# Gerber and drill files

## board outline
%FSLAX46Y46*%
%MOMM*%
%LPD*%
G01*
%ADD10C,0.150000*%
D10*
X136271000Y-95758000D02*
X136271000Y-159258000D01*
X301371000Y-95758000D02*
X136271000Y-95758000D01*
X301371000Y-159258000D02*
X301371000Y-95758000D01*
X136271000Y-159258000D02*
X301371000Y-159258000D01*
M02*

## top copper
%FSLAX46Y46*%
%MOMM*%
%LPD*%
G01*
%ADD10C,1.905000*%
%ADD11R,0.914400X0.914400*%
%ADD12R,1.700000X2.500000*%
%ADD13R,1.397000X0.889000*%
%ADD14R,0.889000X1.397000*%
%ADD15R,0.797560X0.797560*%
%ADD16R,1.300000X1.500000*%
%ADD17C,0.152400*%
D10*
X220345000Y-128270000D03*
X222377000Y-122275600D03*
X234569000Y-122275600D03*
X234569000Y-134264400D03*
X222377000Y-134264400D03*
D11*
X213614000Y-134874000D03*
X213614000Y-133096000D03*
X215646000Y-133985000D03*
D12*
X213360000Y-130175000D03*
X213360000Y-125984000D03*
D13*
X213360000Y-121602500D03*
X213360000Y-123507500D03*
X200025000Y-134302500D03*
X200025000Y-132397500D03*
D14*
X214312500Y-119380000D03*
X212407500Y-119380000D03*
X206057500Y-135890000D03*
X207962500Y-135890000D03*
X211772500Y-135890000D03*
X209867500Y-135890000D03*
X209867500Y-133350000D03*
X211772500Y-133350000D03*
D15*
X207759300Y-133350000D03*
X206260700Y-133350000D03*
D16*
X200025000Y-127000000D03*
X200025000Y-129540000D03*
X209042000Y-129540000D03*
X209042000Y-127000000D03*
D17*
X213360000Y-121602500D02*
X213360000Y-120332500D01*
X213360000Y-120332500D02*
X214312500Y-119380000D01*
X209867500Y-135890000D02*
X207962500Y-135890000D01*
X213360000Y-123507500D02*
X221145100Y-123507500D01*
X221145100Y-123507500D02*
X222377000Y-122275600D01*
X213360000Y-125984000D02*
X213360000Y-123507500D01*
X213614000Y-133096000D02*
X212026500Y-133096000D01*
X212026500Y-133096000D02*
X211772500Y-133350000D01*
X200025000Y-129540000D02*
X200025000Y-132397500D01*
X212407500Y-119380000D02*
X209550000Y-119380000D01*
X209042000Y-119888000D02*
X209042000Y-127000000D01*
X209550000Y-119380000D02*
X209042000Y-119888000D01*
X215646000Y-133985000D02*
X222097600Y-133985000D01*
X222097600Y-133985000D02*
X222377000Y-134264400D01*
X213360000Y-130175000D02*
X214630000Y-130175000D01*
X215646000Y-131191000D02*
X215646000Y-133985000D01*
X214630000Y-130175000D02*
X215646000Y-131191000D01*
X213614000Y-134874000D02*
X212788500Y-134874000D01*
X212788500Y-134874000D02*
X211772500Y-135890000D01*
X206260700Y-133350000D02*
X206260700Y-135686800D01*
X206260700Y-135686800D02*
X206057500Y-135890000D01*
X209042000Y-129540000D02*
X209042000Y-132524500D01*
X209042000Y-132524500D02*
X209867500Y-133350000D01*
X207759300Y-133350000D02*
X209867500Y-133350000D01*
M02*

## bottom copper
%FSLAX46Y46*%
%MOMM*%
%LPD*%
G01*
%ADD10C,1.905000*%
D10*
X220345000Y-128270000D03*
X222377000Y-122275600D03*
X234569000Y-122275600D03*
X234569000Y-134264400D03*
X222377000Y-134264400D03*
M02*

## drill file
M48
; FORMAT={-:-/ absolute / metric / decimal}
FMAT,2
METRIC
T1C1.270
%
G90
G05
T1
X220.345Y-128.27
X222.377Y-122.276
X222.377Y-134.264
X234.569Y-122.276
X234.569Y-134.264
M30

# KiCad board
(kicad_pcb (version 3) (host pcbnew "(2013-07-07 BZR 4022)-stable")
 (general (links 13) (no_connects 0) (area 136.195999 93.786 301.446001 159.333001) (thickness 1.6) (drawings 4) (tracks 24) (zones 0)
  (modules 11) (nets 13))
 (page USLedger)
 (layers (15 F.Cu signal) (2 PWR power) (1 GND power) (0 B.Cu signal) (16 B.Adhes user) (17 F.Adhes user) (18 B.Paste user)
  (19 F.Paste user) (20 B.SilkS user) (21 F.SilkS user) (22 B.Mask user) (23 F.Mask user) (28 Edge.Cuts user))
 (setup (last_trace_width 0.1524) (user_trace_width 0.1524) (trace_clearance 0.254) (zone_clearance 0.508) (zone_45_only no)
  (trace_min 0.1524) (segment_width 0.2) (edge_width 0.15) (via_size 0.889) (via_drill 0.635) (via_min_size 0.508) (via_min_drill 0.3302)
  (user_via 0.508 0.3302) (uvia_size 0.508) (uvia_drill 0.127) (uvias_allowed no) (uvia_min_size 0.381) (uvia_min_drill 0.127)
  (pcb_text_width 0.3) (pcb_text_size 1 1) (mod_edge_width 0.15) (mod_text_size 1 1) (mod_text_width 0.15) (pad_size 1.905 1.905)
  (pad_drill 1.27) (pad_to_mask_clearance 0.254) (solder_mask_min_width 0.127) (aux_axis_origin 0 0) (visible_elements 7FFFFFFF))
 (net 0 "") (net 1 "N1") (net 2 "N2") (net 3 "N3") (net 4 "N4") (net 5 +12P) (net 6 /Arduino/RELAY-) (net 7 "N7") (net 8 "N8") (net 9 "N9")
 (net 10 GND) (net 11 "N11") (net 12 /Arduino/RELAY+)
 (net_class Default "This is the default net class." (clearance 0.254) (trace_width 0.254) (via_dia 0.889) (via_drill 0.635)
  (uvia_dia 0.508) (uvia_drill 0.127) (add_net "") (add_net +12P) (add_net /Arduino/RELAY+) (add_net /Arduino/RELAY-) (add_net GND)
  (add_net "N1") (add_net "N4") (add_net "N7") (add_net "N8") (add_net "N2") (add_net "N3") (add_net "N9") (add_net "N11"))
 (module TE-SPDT (layer F.Cu) (at 220.345 128.27)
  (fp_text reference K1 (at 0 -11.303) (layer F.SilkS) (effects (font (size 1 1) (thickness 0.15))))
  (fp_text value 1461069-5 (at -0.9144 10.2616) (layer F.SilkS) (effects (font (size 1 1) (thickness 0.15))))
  (pad 1 thru_hole circle (at 0 0) (size 1.905 1.905) (drill 1.27) (layers *.Cu *.Mask F.SilkS))
  (pad 2 thru_hole circle (at 2.032 -5.9944) (size 1.905 1.905) (drill 1.27) (layers *.Cu *.Mask F.SilkS) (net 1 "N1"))
  (pad 3 thru_hole circle (at 14.224 -5.9944) (size 1.905 1.905) (drill 1.27) (layers *.Cu *.Mask F.SilkS))
  (pad 4 thru_hole circle (at 14.224 5.9944) (size 1.905 1.905) (drill 1.27) (layers *.Cu *.Mask F.SilkS))
  (pad 5 thru_hole circle (at 2.032 5.9944) (size 1.905 1.905) (drill 1.27) (layers *.Cu *.Mask F.SilkS) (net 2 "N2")))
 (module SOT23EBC (layer F.Cu) (at 214.63 133.985 90)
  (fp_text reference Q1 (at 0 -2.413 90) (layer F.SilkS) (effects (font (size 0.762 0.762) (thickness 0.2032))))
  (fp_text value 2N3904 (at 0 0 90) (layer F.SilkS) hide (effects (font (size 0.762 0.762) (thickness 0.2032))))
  (pad 1 smd rect (at -0.889 -1.016 90) (size 0.9144 0.9144) (layers F.Cu F.Paste F.Mask) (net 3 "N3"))
  (pad 2 smd rect (at 0.889 -1.016 90) (size 0.9144 0.9144) (layers F.Cu F.Paste F.Mask) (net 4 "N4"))
  (pad 3 smd rect (at 0 1.016 90) (size 0.9144 0.9144) (layers F.Cu F.Paste F.Mask) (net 2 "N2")))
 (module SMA (layer F.Cu) (at 213.36 130.175 90)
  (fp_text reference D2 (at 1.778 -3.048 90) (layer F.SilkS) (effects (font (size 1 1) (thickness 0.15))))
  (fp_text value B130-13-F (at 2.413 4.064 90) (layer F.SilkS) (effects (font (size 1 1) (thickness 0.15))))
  (pad 1 smd rect (at 0 0 90) (size 2.5 1.7) (layers F.Cu F.Paste F.Mask) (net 2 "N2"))
  (pad 2 smd rect (at 4.191 0 90) (size 2.5 1.7) (layers F.Cu F.Paste F.Mask) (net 1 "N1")))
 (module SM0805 (layer F.Cu) (at 213.36 122.555 270)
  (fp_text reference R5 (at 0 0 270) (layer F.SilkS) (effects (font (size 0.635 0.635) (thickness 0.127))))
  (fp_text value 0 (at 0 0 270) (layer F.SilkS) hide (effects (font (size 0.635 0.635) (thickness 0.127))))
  (pad 1 smd rect (at -0.9525 0 270) (size 0.889 1.397) (layers F.Cu F.Paste F.Mask) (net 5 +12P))
  (pad 2 smd rect (at 0.9525 0 270) (size 0.889 1.397) (layers F.Cu F.Paste F.Mask) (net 1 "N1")))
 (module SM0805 (layer F.Cu) (at 200.025 133.35 90)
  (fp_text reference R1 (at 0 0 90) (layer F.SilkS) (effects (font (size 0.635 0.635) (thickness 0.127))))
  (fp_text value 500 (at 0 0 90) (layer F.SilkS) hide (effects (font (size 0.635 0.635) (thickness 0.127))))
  (pad 1 smd rect (at -0.9525 0 90) (size 0.889 1.397) (layers F.Cu F.Paste F.Mask) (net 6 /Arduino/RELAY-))
  (pad 2 smd rect (at 0.9525 0 90) (size 0.889 1.397) (layers F.Cu F.Paste F.Mask) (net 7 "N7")))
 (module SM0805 (layer F.Cu) (at 213.36 119.38 180)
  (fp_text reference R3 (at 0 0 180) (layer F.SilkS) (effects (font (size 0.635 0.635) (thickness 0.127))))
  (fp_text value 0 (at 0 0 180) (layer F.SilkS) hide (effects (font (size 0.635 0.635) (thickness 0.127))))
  (pad 1 smd rect (at -0.9525 0 180) (size 0.889 1.397) (layers F.Cu F.Paste F.Mask) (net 5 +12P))
  (pad 2 smd rect (at 0.9525 0 180) (size 0.889 1.397) (layers F.Cu F.Paste F.Mask) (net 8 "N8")))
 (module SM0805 (layer F.Cu) (at 207.01 135.89)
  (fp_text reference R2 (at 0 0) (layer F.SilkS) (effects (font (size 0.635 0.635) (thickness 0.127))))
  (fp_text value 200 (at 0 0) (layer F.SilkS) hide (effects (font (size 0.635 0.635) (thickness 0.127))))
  (pad 1 smd rect (at -0.9525 0) (size 0.889 1.397) (layers F.Cu F.Paste F.Mask) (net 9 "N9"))
  (pad 2 smd rect (at 0.9525 0) (size 0.889 1.397) (layers F.Cu F.Paste F.Mask) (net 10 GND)))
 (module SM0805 (layer F.Cu) (at 210.82 135.89 180)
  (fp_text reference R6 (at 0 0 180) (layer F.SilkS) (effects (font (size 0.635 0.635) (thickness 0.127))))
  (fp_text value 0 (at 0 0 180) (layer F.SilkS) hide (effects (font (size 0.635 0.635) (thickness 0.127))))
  (pad 1 smd rect (at -0.9525 0 180) (size 0.889 1.397) (layers F.Cu F.Paste F.Mask) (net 3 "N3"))
  (pad 2 smd rect (at 0.9525 0 180) (size 0.889 1.397) (layers F.Cu F.Paste F.Mask) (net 10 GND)))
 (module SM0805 (layer F.Cu) (at 210.82 133.35)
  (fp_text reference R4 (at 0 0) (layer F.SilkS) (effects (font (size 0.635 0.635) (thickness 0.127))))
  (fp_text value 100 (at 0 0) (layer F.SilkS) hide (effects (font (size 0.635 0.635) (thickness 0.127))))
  (pad 1 smd rect (at -0.9525 0) (size 0.889 1.397) (layers F.Cu F.Paste F.Mask) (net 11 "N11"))
  (pad 2 smd rect (at 0.9525 0) (size 0.889 1.397) (layers F.Cu F.Paste F.Mask) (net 4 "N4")))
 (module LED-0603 (layer F.Cu) (at 207.01 133.35 180)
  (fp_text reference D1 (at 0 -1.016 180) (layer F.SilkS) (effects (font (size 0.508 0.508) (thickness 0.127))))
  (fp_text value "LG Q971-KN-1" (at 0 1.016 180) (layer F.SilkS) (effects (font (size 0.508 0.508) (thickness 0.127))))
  (pad 1 smd rect (at -0.7493 0 180) (size 0.79756 0.79756) (layers F.Cu F.Paste F.Mask) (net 11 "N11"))
  (pad 2 smd rect (at 0.7493 0 180) (size 0.79756 0.79756) (layers F.Cu F.Paste F.Mask) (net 9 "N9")))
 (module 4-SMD (layer F.Cu) (at 200.025 127 270)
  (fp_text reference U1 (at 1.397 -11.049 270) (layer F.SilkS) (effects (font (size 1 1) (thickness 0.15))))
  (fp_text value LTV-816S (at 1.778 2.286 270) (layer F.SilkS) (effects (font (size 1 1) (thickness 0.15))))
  (pad 1 smd rect (at 0 0 270) (size 1.5 1.3) (layers F.Cu F.Paste F.Mask) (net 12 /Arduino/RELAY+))
  (pad 2 smd rect (at 2.54 0 270) (size 1.5 1.3) (layers F.Cu F.Paste F.Mask) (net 7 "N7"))
  (pad 3 smd rect (at 2.54 -9.017 270) (size 1.5 1.3) (layers F.Cu F.Paste F.Mask) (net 11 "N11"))
  (pad 4 smd rect (at 0 -9.017 270) (size 1.5 1.3) (layers F.Cu F.Paste F.Mask) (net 8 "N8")))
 (gr_line (start 136.271 95.758) (end 136.271 159.258) (angle 90) (layer Edge.Cuts) (width 0.15))
 (gr_line (start 301.371 95.758) (end 136.271 95.758) (angle 90) (layer Edge.Cuts) (width 0.15))
 (gr_line (start 301.371 159.258) (end 301.371 95.758) (angle 90) (layer Edge.Cuts) (width 0.15))
 (gr_line (start 136.271 159.258) (end 301.371 159.258) (angle 90) (layer Edge.Cuts) (width 0.15))
 (segment (start 213.36 121.6025) (end 213.36 120.3325) (width 0.1524) (layer F.Cu) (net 5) (status 400000))
 (segment (start 213.36 120.3325) (end 214.3125 119.38) (width 0.1524) (layer F.Cu) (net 5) (status 800000))
 (segment (start 209.8675 135.89) (end 207.9625 135.89) (width 0.1524) (layer F.Cu) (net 10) (status C00000))
 (segment (start 213.36 123.5075) (end 221.1451 123.5075) (width 0.1524) (layer F.Cu) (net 1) (status 400000))
 (segment (start 221.1451 123.5075) (end 222.377 122.2756) (width 0.1524) (layer F.Cu) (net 1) (status 800000))
 (segment (start 213.36 125.984) (end 213.36 123.5075) (width 0.1524) (layer F.Cu) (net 1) (status C00000))
 (segment (start 213.614 133.096) (end 212.0265 133.096) (width 0.1524) (layer F.Cu) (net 4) (status C00000))
 (segment (start 212.0265 133.096) (end 211.7725 133.35) (width 0.1524) (layer F.Cu) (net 4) (status C00000))
 (segment (start 200.025 129.54) (end 200.025 132.3975) (width 0.1524) (layer F.Cu) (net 7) (status C00000))
 (segment (start 212.4075 119.38) (end 209.55 119.38) (width 0.1524) (layer F.Cu) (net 8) (status 400000))
 (segment (start 209.042 119.888) (end 209.042 127) (width 0.1524) (layer F.Cu) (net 8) (status 800000))
 (segment (start 209.55 119.38) (end 209.042 119.888) (width 0.1524) (layer F.Cu) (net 8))
 (segment (start 215.646 133.985) (end 222.0976 133.985) (width 0.1524) (layer F.Cu) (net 2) (status C00000))
 (segment (start 222.0976 133.985) (end 222.377 134.2644) (width 0.1524) (layer F.Cu) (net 2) (status C00000))
 (segment (start 213.36 130.175) (end 214.63 130.175) (width 0.1524) (layer F.Cu) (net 2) (status 400000))
 (segment (start 215.646 131.191) (end 215.646 133.985) (width 0.1524) (layer F.Cu) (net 2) (status 800000))
 (segment (start 214.63 130.175) (end 215.646 131.191) (width 0.1524) (layer F.Cu) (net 2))
 (segment (start 213.614 134.874) (end 212.7885 134.874) (width 0.1524) (layer F.Cu) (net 3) (status 400000))
 (segment (start 212.7885 134.874) (end 211.7725 135.89) (width 0.1524) (layer F.Cu) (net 3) (status 800000))
 (segment (start 206.2607 133.35) (end 206.2607 135.6868) (width 0.1524) (layer F.Cu) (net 9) (status C00000))
 (segment (start 206.2607 135.6868) (end 206.0575 135.89) (width 0.1524) (layer F.Cu) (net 9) (status C00000))
 (segment (start 209.042 129.54) (end 209.042 132.5245) (width 0.1524) (layer F.Cu) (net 11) (status 400000))
 (segment (start 209.042 132.5245) (end 209.8675 133.35) (width 0.1524) (layer F.Cu) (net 11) (status 800000))
 (segment (start 207.7593 133.35) (end 209.8675 133.35) (width 0.1524) (layer F.Cu) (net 11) (status C00000)))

